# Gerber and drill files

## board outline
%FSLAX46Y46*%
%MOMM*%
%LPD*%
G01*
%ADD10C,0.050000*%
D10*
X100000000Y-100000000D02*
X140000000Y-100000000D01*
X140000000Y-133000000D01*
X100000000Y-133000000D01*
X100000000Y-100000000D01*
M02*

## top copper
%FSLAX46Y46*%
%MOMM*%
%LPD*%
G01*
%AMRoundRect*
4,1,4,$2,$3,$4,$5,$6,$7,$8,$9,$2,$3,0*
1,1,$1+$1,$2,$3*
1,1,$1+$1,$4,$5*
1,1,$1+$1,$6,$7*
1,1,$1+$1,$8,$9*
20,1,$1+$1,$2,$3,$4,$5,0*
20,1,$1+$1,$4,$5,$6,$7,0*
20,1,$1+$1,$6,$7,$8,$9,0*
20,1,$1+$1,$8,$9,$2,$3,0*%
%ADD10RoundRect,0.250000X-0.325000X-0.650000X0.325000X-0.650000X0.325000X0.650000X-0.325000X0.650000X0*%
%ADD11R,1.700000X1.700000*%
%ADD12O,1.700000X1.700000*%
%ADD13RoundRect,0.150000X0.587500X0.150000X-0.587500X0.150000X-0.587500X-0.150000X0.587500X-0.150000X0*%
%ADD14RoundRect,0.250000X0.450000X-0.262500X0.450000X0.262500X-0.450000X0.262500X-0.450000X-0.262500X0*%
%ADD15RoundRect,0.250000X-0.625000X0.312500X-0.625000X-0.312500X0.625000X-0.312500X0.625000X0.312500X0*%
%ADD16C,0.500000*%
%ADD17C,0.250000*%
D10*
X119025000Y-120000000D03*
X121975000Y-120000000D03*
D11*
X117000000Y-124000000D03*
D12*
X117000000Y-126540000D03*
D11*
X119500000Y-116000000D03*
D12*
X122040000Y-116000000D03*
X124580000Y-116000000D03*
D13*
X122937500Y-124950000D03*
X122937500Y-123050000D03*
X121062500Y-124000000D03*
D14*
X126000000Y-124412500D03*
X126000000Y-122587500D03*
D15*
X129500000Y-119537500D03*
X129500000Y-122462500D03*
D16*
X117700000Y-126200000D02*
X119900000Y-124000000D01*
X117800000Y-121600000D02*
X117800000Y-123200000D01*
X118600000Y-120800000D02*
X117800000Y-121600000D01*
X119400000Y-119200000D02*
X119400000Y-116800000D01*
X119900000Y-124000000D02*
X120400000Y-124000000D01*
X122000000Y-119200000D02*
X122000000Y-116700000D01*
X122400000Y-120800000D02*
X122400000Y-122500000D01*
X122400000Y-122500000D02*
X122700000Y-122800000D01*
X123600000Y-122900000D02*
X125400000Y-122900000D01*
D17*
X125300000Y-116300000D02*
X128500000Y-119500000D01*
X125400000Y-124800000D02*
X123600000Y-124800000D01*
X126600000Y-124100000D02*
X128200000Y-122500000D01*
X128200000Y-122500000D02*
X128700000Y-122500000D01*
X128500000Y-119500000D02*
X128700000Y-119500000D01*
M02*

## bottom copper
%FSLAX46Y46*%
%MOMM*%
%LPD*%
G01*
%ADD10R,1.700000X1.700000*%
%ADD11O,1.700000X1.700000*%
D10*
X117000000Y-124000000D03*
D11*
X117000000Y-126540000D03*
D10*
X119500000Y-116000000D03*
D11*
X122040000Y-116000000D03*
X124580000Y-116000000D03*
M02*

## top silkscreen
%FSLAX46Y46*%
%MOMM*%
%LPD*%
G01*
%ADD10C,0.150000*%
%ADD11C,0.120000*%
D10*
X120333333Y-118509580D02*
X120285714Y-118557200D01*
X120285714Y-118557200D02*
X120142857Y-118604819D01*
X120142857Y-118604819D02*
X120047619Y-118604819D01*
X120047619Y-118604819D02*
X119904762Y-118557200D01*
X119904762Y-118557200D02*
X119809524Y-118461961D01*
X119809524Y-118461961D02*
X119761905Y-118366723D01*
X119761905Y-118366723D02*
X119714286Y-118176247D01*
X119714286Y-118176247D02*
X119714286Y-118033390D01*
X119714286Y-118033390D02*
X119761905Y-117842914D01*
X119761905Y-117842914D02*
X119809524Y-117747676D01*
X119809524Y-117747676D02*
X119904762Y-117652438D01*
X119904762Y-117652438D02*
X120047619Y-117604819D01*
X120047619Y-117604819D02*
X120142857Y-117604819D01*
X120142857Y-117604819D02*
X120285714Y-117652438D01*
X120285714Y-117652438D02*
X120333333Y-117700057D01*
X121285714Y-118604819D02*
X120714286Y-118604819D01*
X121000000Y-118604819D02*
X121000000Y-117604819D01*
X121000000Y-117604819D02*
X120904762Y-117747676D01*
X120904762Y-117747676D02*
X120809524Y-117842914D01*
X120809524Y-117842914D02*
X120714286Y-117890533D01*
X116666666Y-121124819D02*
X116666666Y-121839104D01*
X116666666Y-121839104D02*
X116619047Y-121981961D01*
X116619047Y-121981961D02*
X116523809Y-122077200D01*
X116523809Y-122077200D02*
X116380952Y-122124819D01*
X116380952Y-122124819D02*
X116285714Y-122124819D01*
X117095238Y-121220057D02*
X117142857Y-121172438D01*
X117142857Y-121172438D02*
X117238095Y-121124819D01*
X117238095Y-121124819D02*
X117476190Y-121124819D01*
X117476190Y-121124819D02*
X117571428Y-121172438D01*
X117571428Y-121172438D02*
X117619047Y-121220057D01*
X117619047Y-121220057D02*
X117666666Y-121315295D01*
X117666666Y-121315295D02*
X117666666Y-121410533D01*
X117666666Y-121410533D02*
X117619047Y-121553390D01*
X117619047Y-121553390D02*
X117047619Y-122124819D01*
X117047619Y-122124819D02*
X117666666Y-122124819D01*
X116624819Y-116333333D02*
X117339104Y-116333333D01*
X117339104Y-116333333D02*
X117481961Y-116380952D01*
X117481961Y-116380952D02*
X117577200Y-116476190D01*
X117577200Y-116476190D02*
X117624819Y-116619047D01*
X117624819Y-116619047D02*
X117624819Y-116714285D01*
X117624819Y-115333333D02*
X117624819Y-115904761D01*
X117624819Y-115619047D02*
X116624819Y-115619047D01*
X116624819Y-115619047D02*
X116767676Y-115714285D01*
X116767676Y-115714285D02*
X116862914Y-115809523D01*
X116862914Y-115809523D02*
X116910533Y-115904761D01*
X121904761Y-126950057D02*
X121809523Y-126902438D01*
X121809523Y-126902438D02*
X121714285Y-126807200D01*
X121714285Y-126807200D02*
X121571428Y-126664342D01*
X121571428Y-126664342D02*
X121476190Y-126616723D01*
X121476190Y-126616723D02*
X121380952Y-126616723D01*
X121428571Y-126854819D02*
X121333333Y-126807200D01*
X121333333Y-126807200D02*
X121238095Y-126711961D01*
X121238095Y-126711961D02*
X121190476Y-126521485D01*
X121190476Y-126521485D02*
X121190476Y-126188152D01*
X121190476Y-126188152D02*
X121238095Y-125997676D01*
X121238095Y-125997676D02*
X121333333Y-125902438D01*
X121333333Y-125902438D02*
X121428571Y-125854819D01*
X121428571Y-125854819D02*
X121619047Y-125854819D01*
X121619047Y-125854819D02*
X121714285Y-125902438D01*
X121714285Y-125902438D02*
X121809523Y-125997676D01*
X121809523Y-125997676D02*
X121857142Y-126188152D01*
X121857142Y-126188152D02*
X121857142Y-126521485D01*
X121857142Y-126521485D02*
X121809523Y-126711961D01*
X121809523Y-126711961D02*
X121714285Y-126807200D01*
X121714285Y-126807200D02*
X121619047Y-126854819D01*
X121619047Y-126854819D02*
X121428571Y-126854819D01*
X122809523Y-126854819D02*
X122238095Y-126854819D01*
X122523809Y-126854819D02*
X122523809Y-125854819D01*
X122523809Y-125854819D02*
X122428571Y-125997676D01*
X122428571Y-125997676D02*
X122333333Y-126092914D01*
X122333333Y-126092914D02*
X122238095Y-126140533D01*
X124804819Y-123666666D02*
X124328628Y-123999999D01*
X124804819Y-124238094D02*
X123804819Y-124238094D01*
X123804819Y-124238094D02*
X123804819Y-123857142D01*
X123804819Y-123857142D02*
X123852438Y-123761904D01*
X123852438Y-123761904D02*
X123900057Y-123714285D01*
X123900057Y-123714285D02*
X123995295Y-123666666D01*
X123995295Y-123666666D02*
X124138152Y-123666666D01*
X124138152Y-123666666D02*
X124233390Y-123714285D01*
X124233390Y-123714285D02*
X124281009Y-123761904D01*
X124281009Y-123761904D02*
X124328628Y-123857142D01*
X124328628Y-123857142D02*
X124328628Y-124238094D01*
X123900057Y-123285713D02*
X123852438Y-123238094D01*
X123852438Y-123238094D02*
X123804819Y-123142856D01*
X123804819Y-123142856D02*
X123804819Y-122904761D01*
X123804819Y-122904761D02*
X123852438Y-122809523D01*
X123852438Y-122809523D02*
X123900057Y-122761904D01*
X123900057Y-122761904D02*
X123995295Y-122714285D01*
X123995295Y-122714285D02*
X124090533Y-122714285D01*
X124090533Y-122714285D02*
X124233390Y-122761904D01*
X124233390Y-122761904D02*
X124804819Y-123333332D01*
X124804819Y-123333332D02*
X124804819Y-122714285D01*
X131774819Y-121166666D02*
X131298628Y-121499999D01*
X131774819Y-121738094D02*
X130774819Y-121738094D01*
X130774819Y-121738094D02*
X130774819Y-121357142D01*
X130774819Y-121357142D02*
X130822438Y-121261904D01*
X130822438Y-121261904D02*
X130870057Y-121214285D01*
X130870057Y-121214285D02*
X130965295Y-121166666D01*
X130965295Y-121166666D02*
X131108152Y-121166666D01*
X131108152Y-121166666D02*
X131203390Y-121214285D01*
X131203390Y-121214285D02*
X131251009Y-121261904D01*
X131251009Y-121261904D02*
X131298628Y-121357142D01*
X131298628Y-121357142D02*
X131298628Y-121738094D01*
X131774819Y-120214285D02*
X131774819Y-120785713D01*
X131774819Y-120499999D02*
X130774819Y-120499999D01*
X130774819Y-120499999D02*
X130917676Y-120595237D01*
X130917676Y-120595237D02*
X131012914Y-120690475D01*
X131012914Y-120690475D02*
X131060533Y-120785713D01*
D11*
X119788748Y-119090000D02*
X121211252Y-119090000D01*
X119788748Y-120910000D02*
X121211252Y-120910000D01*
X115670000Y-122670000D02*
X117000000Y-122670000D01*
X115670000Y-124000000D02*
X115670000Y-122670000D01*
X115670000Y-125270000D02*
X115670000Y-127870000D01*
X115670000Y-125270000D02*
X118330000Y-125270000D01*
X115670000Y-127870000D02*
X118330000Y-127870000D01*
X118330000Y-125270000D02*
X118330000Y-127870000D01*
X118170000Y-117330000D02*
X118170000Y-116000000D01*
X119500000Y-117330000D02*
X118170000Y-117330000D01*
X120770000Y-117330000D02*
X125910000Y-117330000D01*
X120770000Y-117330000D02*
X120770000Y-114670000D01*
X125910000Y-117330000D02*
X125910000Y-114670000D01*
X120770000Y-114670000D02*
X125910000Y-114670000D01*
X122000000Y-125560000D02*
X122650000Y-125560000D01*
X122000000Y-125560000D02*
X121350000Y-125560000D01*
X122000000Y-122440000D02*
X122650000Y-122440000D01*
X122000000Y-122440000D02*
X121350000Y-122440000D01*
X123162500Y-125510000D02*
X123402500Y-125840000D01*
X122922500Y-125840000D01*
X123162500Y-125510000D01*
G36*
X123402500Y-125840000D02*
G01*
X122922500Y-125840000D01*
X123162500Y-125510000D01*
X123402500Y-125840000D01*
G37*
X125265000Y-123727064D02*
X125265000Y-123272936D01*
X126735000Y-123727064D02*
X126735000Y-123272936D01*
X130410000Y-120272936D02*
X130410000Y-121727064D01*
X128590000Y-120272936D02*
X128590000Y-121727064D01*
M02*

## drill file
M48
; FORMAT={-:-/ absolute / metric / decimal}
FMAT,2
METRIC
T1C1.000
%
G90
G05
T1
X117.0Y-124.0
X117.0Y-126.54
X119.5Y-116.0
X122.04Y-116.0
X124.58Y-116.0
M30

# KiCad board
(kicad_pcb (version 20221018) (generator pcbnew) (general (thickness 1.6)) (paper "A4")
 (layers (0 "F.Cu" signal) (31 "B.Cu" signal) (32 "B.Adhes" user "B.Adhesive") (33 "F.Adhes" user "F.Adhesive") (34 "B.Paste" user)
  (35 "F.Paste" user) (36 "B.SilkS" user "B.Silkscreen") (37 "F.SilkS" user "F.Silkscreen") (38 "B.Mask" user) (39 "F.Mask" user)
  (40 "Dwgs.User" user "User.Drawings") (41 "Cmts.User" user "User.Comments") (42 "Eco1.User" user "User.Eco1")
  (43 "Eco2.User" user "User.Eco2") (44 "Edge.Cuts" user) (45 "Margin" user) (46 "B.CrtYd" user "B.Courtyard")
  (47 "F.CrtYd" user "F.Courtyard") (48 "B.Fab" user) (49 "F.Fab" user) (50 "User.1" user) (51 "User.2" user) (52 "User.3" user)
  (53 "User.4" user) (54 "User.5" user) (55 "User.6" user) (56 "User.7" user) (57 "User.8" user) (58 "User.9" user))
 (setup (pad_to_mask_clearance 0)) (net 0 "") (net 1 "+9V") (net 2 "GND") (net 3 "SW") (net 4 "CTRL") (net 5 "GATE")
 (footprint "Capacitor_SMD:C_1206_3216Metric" (layer "F.Cu") (at 120.5 120)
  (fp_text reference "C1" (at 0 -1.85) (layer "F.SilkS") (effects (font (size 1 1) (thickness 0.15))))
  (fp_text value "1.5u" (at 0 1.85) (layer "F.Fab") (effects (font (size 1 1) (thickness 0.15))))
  (fp_line (start -0.711252 -0.91) (end 0.711252 -0.91) (stroke (width 0.12) (type solid)) (layer "F.SilkS"))
  (fp_line (start -0.711252 0.91) (end 0.711252 0.91) (stroke (width 0.12) (type solid)) (layer "F.SilkS"))
  (pad "1" smd roundrect (at -1.475 0) (size 1.15 1.8) (layers "F.Cu" "F.Paste" "F.Mask") (roundrect_rratio 0.217391) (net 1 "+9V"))
  (pad "2" smd roundrect (at 1.475 0) (size 1.15 1.8) (layers "F.Cu" "F.Paste" "F.Mask") (roundrect_rratio 0.217391) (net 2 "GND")))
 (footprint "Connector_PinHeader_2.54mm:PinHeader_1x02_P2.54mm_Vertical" (layer "F.Cu") (at 117 124)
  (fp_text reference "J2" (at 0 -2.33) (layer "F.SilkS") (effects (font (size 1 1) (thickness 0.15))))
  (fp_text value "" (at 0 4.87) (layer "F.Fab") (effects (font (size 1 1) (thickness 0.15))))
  (fp_line (start -1.33 -1.33) (end 0 -1.33) (stroke (width 0.12) (type solid)) (layer "F.SilkS"))
  (fp_line (start -1.33 0) (end -1.33 -1.33) (stroke (width 0.12) (type solid)) (layer "F.SilkS"))
  (fp_line (start -1.33 1.27) (end -1.33 3.87) (stroke (width 0.12) (type solid)) (layer "F.SilkS"))
  (fp_line (start -1.33 1.27) (end 1.33 1.27) (stroke (width 0.12) (type solid)) (layer "F.SilkS"))
  (fp_line (start -1.33 3.87) (end 1.33 3.87) (stroke (width 0.12) (type solid)) (layer "F.SilkS"))
  (fp_line (start 1.33 1.27) (end 1.33 3.87) (stroke (width 0.12) (type solid)) (layer "F.SilkS"))
  (pad "1" thru_hole rect (at 0 0) (size 1.7 1.7) (drill 1) (layers "*.Cu" "*.Mask") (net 1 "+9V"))
  (pad "2" thru_hole oval (at 0 2.54) (size 1.7 1.7) (drill 1) (layers "*.Cu" "*.Mask") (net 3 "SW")))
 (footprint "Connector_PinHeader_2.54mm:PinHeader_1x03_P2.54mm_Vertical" (layer "F.Cu") (at 119.5 116 90)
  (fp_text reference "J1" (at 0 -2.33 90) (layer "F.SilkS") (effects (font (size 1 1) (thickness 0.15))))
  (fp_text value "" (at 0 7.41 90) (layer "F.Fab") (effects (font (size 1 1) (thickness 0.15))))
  (fp_line (start -1.33 -1.33) (end 0 -1.33) (stroke (width 0.12) (type solid)) (layer "F.SilkS"))
  (fp_line (start -1.33 0) (end -1.33 -1.33) (stroke (width 0.12) (type solid)) (layer "F.SilkS"))
  (fp_line (start -1.33 1.27) (end -1.33 6.41) (stroke (width 0.12) (type solid)) (layer "F.SilkS"))
  (fp_line (start -1.33 1.27) (end 1.33 1.27) (stroke (width 0.12) (type solid)) (layer "F.SilkS"))
  (fp_line (start -1.33 6.41) (end 1.33 6.41) (stroke (width 0.12) (type solid)) (layer "F.SilkS"))
  (fp_line (start 1.33 1.27) (end 1.33 6.41) (stroke (width 0.12) (type solid)) (layer "F.SilkS"))
  (pad "1" thru_hole rect (at 0 0 90) (size 1.7 1.7) (drill 1) (layers "*.Cu" "*.Mask") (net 1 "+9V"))
  (pad "2" thru_hole oval (at 0 2.54 90) (size 1.7 1.7) (drill 1) (layers "*.Cu" "*.Mask") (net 2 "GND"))
  (pad "3" thru_hole oval (at 0 5.08 90) (size 1.7 1.7) (drill 1) (layers "*.Cu" "*.Mask") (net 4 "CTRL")))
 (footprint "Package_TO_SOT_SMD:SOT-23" (layer "F.Cu") (at 122 124 180)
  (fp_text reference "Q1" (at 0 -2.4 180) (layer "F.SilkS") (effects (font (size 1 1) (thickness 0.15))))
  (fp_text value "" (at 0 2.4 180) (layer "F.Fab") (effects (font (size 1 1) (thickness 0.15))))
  (fp_line (start 0 -1.56) (end -0.65 -1.56) (stroke (width 0.12) (type solid)) (layer "F.SilkS"))
  (fp_line (start 0 -1.56) (end 0.65 -1.56) (stroke (width 0.12) (type solid)) (layer "F.SilkS"))
  (fp_line (start 0 1.56) (end -0.65 1.56) (stroke (width 0.12) (type solid)) (layer "F.SilkS"))
  (fp_line (start 0 1.56) (end 0.65 1.56) (stroke (width 0.12) (type solid)) (layer "F.SilkS"))
  (fp_poly
   (pts (xy -1.1625 -1.51) (xy -1.4025 -1.84) (xy -0.9225 -1.84) (xy -1.1625 -1.51)) (stroke (width 0.12) (type solid)) (fill solid)
   (layer "F.SilkS"))
  (pad "1" smd roundrect (at -0.9375 -0.95 180) (size 1.475 0.6) (layers "F.Cu" "F.Paste" "F.Mask") (roundrect_rratio 0.25) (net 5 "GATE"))
  (pad "2" smd roundrect (at -0.9375 0.95 180) (size 1.475 0.6) (layers "F.Cu" "F.Paste" "F.Mask") (roundrect_rratio 0.25) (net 2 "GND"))
  (pad "3" smd roundrect (at 0.9375 0 180) (size 1.475 0.6) (layers "F.Cu" "F.Paste" "F.Mask") (roundrect_rratio 0.25) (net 3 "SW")))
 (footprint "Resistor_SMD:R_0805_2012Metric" (layer "F.Cu") (at 126 123.5 90)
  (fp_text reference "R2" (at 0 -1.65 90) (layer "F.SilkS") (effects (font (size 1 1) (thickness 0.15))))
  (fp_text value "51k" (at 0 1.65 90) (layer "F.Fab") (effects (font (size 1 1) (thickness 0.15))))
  (fp_line (start -0.227064 -0.735) (end 0.227064 -0.735) (stroke (width 0.12) (type solid)) (layer "F.SilkS"))
  (fp_line (start -0.227064 0.735) (end 0.227064 0.735) (stroke (width 0.12) (type solid)) (layer "F.SilkS"))
  (pad "1" smd roundrect (at -0.9125 0 90) (size 1.025 1.4) (layers "F.Cu" "F.Paste" "F.Mask") (roundrect_rratio 0.243902) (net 5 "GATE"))
  (pad "2" smd roundrect (at 0.9125 0 90) (size 1.025 1.4) (layers "F.Cu" "F.Paste" "F.Mask") (roundrect_rratio 0.243902) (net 2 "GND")))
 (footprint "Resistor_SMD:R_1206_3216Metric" (layer "F.Cu") (at 129.5 121 -90)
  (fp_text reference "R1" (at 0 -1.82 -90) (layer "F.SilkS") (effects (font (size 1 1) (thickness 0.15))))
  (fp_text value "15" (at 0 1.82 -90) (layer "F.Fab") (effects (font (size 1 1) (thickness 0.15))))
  (fp_line (start -0.727064 -0.91) (end 0.727064 -0.91) (stroke (width 0.12) (type solid)) (layer "F.SilkS"))
  (fp_line (start -0.727064 0.91) (end 0.727064 0.91) (stroke (width 0.12) (type solid)) (layer "F.SilkS"))
  (pad "1" smd roundrect (at -1.4625 0 270) (size 1.125 1.75) (layers "F.Cu" "F.Paste" "F.Mask") (roundrect_rratio 0.222222) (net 4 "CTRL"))
  (pad "2" smd roundrect (at 1.4625 0 270) (size 1.125 1.75) (layers "F.Cu" "F.Paste" "F.Mask") (roundrect_rratio 0.222222) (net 5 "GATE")))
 (gr_rect (start 100 100) (end 140 133) (stroke (width 0.05) (type default)) (fill none) (layer "Edge.Cuts"))
 (segment (start 117.7 126.2) (end 119.9 124) (width 0.5) (layer "F.Cu") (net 3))
 (segment (start 117.8 121.6) (end 117.8 123.2) (width 0.5) (layer "F.Cu") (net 1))
 (segment (start 118.6 120.8) (end 117.8 121.6) (width 0.5) (layer "F.Cu") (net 1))
 (segment (start 119.4 119.2) (end 119.4 116.8) (width 0.5) (layer "F.Cu") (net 1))
 (segment (start 119.9 124) (end 120.4 124) (width 0.5) (layer "F.Cu") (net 3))
 (segment (start 122 119.2) (end 122 116.7) (width 0.5) (layer "F.Cu") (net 2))
 (segment (start 122.4 120.8) (end 122.4 122.5) (width 0.5) (layer "F.Cu") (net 2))
 (segment (start 122.4 122.5) (end 122.7 122.8) (width 0.5) (layer "F.Cu") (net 2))
 (segment (start 123.6 122.9) (end 125.4 122.9) (width 0.5) (layer "F.Cu") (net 2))
 (segment (start 125.3 116.3) (end 128.5 119.5) (width 0.25) (layer "F.Cu") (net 4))
 (segment (start 125.4 124.8) (end 123.6 124.8) (width 0.25) (layer "F.Cu") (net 5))
 (segment (start 126.6 124.1) (end 128.2 122.5) (width 0.25) (layer "F.Cu") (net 5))
 (segment (start 128.2 122.5) (end 128.7 122.5) (width 0.25) (layer "F.Cu") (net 5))
 (segment (start 128.5 119.5) (end 128.7 119.5) (width 0.25) (layer "F.Cu") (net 4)))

